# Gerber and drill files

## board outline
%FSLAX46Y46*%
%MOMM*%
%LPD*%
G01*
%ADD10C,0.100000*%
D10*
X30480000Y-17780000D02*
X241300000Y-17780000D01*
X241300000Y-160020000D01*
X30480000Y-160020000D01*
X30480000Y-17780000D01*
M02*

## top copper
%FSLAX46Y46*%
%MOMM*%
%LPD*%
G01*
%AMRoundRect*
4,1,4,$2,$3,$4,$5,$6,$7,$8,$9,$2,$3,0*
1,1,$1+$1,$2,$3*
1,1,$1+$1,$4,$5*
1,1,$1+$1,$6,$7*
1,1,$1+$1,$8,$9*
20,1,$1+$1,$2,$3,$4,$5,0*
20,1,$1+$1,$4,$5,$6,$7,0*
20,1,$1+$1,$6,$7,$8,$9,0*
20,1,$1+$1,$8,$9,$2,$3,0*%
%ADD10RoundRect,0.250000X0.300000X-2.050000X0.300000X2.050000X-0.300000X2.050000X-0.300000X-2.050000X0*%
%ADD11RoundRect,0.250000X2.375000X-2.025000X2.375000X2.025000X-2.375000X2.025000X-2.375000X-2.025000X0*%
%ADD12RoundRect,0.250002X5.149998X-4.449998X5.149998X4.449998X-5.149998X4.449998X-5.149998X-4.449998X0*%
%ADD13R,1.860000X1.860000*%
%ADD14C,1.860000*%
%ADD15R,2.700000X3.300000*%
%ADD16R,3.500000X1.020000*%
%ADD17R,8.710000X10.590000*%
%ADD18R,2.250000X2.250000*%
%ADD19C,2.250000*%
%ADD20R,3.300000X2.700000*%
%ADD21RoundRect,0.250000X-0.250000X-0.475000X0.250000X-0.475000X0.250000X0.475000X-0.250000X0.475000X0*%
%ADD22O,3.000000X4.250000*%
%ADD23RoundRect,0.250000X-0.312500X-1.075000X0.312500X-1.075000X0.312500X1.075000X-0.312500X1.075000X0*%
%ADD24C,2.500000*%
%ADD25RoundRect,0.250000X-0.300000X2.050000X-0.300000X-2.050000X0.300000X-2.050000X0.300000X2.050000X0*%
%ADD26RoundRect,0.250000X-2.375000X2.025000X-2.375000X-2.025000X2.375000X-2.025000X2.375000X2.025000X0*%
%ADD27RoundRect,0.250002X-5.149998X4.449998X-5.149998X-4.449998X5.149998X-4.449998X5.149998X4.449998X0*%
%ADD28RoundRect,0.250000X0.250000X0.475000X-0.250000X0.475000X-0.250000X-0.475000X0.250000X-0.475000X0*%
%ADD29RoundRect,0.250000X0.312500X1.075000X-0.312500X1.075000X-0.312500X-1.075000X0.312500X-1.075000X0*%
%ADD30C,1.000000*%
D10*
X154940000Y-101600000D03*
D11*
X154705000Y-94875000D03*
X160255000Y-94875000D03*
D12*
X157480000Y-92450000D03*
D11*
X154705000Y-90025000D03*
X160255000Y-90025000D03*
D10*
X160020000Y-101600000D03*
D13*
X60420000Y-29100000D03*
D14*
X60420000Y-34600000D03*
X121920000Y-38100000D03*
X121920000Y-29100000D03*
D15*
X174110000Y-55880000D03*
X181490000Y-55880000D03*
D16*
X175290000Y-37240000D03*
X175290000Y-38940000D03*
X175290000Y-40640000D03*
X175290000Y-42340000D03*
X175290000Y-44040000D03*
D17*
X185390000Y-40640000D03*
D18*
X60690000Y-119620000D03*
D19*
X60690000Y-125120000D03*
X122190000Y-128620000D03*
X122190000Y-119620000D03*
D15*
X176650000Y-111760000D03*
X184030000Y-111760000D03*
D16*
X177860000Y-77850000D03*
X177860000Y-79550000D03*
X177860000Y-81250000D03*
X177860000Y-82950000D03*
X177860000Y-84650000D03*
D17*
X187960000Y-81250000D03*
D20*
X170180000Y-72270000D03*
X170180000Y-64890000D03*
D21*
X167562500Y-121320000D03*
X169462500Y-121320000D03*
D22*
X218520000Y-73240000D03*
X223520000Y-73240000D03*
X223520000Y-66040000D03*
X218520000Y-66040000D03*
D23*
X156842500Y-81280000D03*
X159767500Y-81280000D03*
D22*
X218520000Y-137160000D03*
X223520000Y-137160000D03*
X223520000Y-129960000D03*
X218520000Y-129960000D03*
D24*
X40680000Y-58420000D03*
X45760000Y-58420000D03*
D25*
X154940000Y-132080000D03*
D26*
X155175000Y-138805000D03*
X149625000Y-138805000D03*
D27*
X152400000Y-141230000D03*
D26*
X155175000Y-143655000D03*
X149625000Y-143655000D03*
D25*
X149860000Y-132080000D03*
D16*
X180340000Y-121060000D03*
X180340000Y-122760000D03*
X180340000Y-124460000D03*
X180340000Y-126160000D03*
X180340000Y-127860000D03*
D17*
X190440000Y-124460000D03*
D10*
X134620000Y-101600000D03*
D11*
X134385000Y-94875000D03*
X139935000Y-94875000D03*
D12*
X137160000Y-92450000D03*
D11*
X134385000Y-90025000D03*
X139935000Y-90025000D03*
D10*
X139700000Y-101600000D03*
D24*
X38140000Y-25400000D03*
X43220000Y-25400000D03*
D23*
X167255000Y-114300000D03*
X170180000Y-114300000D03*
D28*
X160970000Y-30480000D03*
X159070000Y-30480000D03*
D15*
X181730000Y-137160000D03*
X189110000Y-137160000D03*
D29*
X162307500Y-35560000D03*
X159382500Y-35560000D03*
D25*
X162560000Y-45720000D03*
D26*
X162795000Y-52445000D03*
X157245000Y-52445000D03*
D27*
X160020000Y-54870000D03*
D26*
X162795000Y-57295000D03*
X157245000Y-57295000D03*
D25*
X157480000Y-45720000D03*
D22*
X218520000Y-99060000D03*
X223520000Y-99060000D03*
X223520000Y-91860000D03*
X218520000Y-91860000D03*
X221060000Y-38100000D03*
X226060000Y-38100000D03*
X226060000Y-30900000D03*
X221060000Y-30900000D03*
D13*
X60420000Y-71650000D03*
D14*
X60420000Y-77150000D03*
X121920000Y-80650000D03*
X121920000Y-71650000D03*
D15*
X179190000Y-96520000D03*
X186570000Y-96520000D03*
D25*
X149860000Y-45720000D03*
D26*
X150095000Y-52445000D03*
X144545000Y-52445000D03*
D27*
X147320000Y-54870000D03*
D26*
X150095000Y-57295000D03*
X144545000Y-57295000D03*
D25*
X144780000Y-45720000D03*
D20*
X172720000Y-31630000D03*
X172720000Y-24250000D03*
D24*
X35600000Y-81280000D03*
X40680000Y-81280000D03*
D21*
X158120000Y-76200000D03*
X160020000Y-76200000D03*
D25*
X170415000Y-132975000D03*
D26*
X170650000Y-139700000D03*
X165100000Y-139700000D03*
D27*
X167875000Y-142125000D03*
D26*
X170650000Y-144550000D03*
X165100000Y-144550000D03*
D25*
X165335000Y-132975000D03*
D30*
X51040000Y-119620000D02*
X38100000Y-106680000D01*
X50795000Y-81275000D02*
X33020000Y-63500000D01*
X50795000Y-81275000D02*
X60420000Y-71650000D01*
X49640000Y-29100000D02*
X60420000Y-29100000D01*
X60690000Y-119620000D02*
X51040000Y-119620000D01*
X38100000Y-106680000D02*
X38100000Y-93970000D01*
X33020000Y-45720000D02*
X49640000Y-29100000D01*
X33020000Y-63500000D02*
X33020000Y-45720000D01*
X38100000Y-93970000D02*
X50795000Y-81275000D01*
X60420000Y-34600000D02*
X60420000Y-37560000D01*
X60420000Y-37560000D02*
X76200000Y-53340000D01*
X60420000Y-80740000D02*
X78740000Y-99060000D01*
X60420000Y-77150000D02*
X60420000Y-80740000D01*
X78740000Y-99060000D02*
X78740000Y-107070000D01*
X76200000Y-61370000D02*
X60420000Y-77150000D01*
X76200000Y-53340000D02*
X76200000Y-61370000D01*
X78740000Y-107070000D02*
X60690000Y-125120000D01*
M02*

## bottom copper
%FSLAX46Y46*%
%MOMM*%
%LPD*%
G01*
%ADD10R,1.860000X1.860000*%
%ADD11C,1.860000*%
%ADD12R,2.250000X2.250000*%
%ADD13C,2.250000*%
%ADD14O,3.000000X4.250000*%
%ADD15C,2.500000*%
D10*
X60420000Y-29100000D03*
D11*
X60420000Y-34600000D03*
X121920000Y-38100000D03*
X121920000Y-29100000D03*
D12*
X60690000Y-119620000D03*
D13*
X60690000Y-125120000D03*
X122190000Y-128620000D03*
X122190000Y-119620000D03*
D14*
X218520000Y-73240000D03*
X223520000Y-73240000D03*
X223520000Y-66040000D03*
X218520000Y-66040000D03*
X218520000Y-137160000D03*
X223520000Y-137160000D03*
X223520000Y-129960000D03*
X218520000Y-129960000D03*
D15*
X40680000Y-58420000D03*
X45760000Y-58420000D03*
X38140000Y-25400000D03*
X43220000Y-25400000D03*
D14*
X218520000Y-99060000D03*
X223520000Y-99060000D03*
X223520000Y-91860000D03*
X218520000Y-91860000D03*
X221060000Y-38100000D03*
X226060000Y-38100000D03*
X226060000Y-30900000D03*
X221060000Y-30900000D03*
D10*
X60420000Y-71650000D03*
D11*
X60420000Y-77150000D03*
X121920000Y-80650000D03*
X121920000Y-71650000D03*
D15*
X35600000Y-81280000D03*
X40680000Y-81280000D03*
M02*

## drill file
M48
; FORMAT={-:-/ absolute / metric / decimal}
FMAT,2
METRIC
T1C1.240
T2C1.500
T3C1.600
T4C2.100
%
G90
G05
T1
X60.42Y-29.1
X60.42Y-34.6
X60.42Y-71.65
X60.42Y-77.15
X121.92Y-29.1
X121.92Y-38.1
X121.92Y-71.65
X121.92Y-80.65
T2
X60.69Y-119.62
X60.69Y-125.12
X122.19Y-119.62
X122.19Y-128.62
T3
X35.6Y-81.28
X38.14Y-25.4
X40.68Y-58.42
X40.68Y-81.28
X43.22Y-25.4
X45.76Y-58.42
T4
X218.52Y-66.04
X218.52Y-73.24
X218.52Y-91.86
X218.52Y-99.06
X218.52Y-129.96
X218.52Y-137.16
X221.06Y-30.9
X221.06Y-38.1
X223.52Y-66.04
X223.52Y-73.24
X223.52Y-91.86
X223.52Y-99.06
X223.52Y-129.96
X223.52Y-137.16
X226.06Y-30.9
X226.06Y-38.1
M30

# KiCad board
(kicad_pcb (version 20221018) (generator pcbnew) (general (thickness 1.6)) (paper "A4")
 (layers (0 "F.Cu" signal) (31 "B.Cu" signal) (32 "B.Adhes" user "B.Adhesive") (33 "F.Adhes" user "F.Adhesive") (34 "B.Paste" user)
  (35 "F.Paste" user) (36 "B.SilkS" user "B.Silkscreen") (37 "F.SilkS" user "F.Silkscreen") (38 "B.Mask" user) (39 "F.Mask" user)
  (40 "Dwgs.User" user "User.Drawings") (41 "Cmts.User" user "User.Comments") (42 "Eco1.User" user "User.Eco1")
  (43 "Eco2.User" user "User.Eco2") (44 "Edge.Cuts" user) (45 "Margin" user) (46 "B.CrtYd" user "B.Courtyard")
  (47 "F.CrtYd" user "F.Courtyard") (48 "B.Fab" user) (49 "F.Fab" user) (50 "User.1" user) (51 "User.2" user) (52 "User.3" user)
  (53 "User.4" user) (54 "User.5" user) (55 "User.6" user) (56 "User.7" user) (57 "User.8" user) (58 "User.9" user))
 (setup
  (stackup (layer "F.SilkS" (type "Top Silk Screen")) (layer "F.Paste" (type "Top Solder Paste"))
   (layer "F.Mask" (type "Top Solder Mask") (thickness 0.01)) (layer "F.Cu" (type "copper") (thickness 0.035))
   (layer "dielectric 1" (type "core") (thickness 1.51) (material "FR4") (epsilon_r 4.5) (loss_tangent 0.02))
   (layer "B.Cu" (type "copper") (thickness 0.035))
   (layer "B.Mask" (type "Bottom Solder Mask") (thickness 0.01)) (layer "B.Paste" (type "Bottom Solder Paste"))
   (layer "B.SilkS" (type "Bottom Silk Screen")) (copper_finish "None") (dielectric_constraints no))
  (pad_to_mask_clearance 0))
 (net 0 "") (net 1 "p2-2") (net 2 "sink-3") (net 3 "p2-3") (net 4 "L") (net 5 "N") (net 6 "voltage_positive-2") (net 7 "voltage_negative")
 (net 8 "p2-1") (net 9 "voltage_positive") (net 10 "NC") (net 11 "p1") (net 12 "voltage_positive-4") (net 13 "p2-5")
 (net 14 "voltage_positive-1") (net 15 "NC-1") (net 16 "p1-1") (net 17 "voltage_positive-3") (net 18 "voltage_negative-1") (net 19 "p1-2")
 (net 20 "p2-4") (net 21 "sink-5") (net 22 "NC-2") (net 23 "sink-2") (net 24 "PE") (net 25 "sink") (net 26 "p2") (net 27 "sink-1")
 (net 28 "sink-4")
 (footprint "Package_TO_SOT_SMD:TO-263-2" (layer "F.Cu") (at 157.48 93.95 90)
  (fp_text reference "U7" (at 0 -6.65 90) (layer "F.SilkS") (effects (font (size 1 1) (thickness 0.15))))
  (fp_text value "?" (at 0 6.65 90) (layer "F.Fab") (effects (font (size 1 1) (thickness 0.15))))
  (pad "1" smd roundrect (at -7.65 -2.54 90) (size 4.6 1.1) (layers "F.Cu" "F.Paste" "F.Mask") (roundrect_rratio 0.227273) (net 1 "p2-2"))
  (pad "2" smd roundrect (at -0.925 -2.775 90) (size 4.55 5.25) (layers "F.Cu" "F.Paste") (roundrect_rratio 0.054945) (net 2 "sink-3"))
  (pad "2" smd roundrect (at -0.925 2.775 90) (size 4.55 5.25) (layers "F.Cu" "F.Paste") (roundrect_rratio 0.054945) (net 2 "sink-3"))
  (pad "2" smd roundrect (at 1.5 0 90) (size 9.4 10.8) (layers "F.Cu" "F.Mask") (roundrect_rratio 0.026596) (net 2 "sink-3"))
  (pad "2" smd roundrect (at 3.925 -2.775 90) (size 4.55 5.25) (layers "F.Cu" "F.Paste") (roundrect_rratio 0.054945) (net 2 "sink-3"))
  (pad "2" smd roundrect (at 3.925 2.775 90) (size 4.55 5.25) (layers "F.Cu" "F.Paste") (roundrect_rratio 0.054945) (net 2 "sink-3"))
  (pad "3" smd roundrect (at -7.65 2.54 90) (size 4.6 1.1) (layers "F.Cu" "F.Paste" "F.Mask") (roundrect_rratio 0.227273) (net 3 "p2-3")))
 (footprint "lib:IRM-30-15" (layer "F.Cu") (at 91.17 44.1)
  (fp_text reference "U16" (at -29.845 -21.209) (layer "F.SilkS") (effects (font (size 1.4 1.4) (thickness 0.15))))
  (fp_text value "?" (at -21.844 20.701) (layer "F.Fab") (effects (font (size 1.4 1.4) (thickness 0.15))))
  (pad "1" thru_hole rect (at -30.75 -15) (size 1.86 1.86) (drill 1.24) (layers "*.Cu" "*.Mask") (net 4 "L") (solder_mask_margin 0.102))
  (pad "2" thru_hole circle (at -30.75 -9.5) (size 1.86 1.86) (drill 1.24) (layers "*.Cu" "*.Mask") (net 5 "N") (solder_mask_margin 0.102))
  (pad "3" thru_hole circle (at 30.75 -6) (size 1.86 1.86) (drill 1.24) (layers "*.Cu" "*.Mask") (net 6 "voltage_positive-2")
   (solder_mask_margin 0.102))
  (pad "4" thru_hole circle (at 30.75 -15) (size 1.86 1.86) (drill 1.24) (layers "*.Cu" "*.Mask") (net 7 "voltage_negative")
   (solder_mask_margin 0.102)))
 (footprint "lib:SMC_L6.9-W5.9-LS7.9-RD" (layer "F.Cu") (at 177.8 55.88)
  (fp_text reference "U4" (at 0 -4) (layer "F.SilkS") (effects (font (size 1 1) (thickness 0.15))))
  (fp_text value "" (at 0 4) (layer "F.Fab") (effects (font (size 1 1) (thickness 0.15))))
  (pad "1" smd rect (at -3.69 0) (size 2.7 3.3) (layers "F.Cu" "F.Paste" "F.Mask") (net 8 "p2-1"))
  (pad "2" smd rect (at 3.69 0) (size 2.7 3.3) (layers "F.Cu" "F.Paste" "F.Mask") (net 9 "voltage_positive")))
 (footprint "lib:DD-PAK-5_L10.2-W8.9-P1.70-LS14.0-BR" (layer "F.Cu") (at 180.34 40.64 180)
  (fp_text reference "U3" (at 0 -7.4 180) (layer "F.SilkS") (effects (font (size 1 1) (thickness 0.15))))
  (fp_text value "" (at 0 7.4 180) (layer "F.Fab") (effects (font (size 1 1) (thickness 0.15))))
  (pad "1" smd rect (at 5.05 3.4 180) (size 3.5 1.02) (layers "F.Cu" "F.Paste" "F.Mask") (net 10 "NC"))
  (pad "2" smd rect (at 5.05 1.7 180) (size 3.5 1.02) (layers "F.Cu" "F.Paste" "F.Mask") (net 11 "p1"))
  (pad "3" smd rect (at 5.05 0 180) (size 3.5 1.02) (layers "F.Cu" "F.Paste" "F.Mask") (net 9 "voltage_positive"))
  (pad "4" smd rect (at 5.05 -1.7 180) (size 3.5 1.02) (layers "F.Cu" "F.Paste" "F.Mask") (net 6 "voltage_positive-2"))
  (pad "5" smd rect (at 5.05 -3.4 180) (size 3.5 1.02) (layers "F.Cu" "F.Paste" "F.Mask") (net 8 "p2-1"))
  (pad "6" smd rect (at -5.05 0) (size 8.71 10.59) (layers "F.Cu" "F.Paste" "F.Mask") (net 9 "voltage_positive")))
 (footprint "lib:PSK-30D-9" (layer "F.Cu") (at 91.44 134.62)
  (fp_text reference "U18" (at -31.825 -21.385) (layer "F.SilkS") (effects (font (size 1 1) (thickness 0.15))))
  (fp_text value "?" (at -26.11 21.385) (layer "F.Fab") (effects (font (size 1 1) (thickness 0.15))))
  (pad "1" thru_hole rect (at -30.75 -15) (size 2.25 2.25) (drill 1.5) (layers "*.Cu" "*.Mask") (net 4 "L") (solder_mask_margin 0.102))
  (pad "2" thru_hole circle (at -30.75 -9.5) (size 2.25 2.25) (drill 1.5) (layers "*.Cu" "*.Mask") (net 5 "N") (solder_mask_margin 0.102))
  (pad "3" thru_hole circle (at 30.75 -6) (size 2.25 2.25) (drill 1.5) (layers "*.Cu" "*.Mask") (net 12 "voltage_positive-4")
   (solder_mask_margin 0.102))
  (pad "4" thru_hole circle (at 30.75 -15) (size 2.25 2.25) (drill 1.5) (layers "*.Cu" "*.Mask") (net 7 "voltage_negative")
   (solder_mask_margin 0.102)))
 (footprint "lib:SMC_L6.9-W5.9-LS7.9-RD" (layer "F.Cu") (at 180.34 111.76)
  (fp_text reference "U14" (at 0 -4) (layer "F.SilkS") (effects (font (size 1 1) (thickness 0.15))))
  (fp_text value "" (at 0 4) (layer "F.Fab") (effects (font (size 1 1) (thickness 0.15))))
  (pad "1" smd rect (at -3.69 0) (size 2.7 3.3) (layers "F.Cu" "F.Paste" "F.Mask") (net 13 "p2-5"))
  (pad "2" smd rect (at 3.69 0) (size 2.7 3.3) (layers "F.Cu" "F.Paste" "F.Mask") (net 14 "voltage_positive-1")))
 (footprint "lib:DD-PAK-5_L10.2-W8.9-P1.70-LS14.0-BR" (layer "F.Cu") (at 182.91 81.25 180)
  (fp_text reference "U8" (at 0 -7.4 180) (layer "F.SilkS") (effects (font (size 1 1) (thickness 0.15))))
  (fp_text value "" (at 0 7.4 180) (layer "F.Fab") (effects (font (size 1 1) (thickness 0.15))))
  (pad "1" smd rect (at 5.05 3.4 180) (size 3.5 1.02) (layers "F.Cu" "F.Paste" "F.Mask") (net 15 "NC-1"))
  (pad "2" smd rect (at 5.05 1.7 180) (size 3.5 1.02) (layers "F.Cu" "F.Paste" "F.Mask") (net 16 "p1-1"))
  (pad "3" smd rect (at 5.05 0 180) (size 3.5 1.02) (layers "F.Cu" "F.Paste" "F.Mask") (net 7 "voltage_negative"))
  (pad "4" smd rect (at 5.05 -1.7 180) (size 3.5 1.02) (layers "F.Cu" "F.Paste" "F.Mask") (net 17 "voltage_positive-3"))
  (pad "5" smd rect (at 5.05 -3.4 180) (size 3.5 1.02) (layers "F.Cu" "F.Paste" "F.Mask") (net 3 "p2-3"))
  (pad "6" smd rect (at -5.05 0) (size 8.71 10.59) (layers "F.Cu" "F.Paste" "F.Mask") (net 7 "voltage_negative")))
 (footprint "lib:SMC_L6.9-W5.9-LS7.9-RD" (layer "F.Cu") (at 170.18 68.58 90)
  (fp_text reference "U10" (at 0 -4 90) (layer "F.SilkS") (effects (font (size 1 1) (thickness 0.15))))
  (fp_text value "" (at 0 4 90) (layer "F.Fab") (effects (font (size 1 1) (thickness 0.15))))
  (pad "1" smd rect (at -3.69 0 90) (size 2.7 3.3) (layers "F.Cu" "F.Paste" "F.Mask") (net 7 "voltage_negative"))
  (pad "2" smd rect (at 3.69 0 90) (size 2.7 3.3) (layers "F.Cu" "F.Paste" "F.Mask") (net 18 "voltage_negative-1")))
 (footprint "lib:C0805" (layer "F.Cu") (at 168.5125 121.32)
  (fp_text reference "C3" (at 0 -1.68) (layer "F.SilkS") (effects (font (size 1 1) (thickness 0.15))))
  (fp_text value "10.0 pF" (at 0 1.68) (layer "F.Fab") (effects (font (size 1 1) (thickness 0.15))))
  (pad "1" smd roundrect (at -0.95 0) (size 1 1.45) (layers "F.Cu" "F.Paste" "F.Mask") (roundrect_rratio 0.25) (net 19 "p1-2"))
  (pad "2" smd roundrect (at 0.95 0) (size 1 1.45) (layers "F.Cu" "F.Paste" "F.Mask") (roundrect_rratio 0.25) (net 7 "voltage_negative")))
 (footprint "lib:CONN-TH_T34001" (layer "F.Cu") (at 221.02 69.64)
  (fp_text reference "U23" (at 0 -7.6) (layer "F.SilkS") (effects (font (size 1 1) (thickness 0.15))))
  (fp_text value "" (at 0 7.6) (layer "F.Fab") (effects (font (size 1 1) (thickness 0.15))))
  (pad "1" thru_hole oval (at -2.5 3.6) (size 3 4.25) (drill 2.100021) (layers "*.Cu" "*.Mask") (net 18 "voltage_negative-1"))
  (pad "2" thru_hole oval (at 2.5 3.6) (size 3 4.25) (drill 2.100021) (layers "*.Cu" "*.Mask") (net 18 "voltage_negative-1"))
  (pad "3" thru_hole oval (at 2.5 -3.6) (size 3 4.25) (drill 2.100021) (layers "*.Cu" "*.Mask") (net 18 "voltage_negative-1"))
  (pad "4" thru_hole oval (at -2.5 -3.6) (size 3 4.25) (drill 2.100021) (layers "*.Cu" "*.Mask") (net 18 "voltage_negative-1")))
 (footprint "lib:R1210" (layer "F.Cu") (at 158.305 81.28)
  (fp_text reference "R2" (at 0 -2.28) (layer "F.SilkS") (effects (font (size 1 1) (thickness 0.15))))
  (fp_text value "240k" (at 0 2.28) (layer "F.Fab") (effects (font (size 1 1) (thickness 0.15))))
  (pad "1" smd roundrect (at -1.4625 0) (size 1.125 2.65) (layers "F.Cu" "F.Paste" "F.Mask") (roundrect_rratio 0.222222) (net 16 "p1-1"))
  (pad "2" smd roundrect (at 1.4625 0) (size 1.125 2.65) (layers "F.Cu" "F.Paste" "F.Mask") (roundrect_rratio 0.222222)
   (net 18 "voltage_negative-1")))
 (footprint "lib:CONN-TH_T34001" (layer "F.Cu") (at 221.02 133.56)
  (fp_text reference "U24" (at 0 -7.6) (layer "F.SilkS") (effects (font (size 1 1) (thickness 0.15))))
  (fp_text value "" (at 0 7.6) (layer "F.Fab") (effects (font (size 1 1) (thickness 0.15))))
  (pad "1" thru_hole oval (at -2.5 3.6) (size 3 4.25) (drill 2.100021) (layers "*.Cu" "*.Mask") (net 14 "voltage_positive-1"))
  (pad "2" thru_hole oval (at 2.5 3.6) (size 3 4.25) (drill 2.100021) (layers "*.Cu" "*.Mask") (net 14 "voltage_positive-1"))
  (pad "3" thru_hole oval (at 2.5 -3.6) (size 3 4.25) (drill 2.100021) (layers "*.Cu" "*.Mask") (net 14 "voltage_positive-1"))
  (pad "4" thru_hole oval (at -2.5 -3.6) (size 3 4.25) (drill 2.100021) (layers "*.Cu" "*.Mask") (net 14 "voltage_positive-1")))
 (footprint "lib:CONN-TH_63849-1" (layer "F.Cu") (at 43.22 58.42)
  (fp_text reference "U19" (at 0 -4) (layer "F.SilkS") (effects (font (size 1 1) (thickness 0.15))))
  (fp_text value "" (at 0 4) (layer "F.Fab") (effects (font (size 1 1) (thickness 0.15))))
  (pad "1" thru_hole circle (at -2.54 0) (size 2.5 2.5) (drill 1.599997) (layers "*.Cu" "*.Mask") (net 4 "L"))
  (pad "1" thru_hole circle (at 2.54 0) (size 2.5 2.5) (drill 1.599997) (layers "*.Cu" "*.Mask") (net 4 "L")))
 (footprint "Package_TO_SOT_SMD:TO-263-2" (layer "F.Cu") (at 152.4 139.73 -90)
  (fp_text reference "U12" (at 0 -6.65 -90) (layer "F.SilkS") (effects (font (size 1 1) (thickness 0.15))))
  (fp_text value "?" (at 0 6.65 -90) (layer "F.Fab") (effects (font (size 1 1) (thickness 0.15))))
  (pad "1" smd roundrect (at -7.65 -2.54 270) (size 4.6 1.1) (layers "F.Cu" "F.Paste" "F.Mask") (roundrect_rratio 0.227273) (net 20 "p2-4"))
  (pad "2" smd roundrect (at -0.925 -2.775 270) (size 4.55 5.25) (layers "F.Cu" "F.Paste") (roundrect_rratio 0.054945) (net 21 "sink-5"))
  (pad "2" smd roundrect (at -0.925 2.775 270) (size 4.55 5.25) (layers "F.Cu" "F.Paste") (roundrect_rratio 0.054945) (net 21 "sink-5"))
  (pad "2" smd roundrect (at 1.5 0 270) (size 9.4 10.8) (layers "F.Cu" "F.Mask") (roundrect_rratio 0.026596) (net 21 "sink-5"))
  (pad "2" smd roundrect (at 3.925 -2.775 270) (size 4.55 5.25) (layers "F.Cu" "F.Paste") (roundrect_rratio 0.054945) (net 21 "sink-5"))
  (pad "2" smd roundrect (at 3.925 2.775 270) (size 4.55 5.25) (layers "F.Cu" "F.Paste") (roundrect_rratio 0.054945) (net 21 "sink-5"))
  (pad "3" smd roundrect (at -7.65 2.54 270) (size 4.6 1.1) (layers "F.Cu" "F.Paste" "F.Mask") (roundrect_rratio 0.227273) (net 13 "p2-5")))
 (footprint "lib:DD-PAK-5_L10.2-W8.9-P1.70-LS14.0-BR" (layer "F.Cu") (at 185.39 124.46 180)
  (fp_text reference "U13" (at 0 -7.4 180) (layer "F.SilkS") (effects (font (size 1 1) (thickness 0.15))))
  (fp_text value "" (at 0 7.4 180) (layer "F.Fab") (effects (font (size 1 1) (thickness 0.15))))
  (pad "1" smd rect (at 5.05 3.4 180) (size 3.5 1.02) (layers "F.Cu" "F.Paste" "F.Mask") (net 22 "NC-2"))
  (pad "2" smd rect (at 5.05 1.7 180) (size 3.5 1.02) (layers "F.Cu" "F.Paste" "F.Mask") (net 19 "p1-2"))
  (pad "3" smd rect (at 5.05 0 180) (size 3.5 1.02) (layers "F.Cu" "F.Paste" "F.Mask") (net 14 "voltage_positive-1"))
  (pad "4" smd rect (at 5.05 -1.7 180) (size 3.5 1.02) (layers "F.Cu" "F.Paste" "F.Mask") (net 12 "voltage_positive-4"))
  (pad "5" smd rect (at 5.05 -3.4 180) (size 3.5 1.02) (layers "F.Cu" "F.Paste" "F.Mask") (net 13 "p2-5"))
  (pad "6" smd rect (at -5.05 0) (size 8.71 10.59) (layers "F.Cu" "F.Paste" "F.Mask") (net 14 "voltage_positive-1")))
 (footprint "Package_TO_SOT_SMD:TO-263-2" (layer "F.Cu") (at 137.16 93.95 90)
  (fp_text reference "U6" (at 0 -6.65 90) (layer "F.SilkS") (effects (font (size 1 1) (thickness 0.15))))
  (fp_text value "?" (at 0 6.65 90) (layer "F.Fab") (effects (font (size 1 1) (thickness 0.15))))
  (pad "1" smd roundrect (at -7.65 -2.54 90) (size 4.6 1.1) (layers "F.Cu" "F.Paste" "F.Mask") (roundrect_rratio 0.227273)
   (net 17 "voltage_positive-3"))
  (pad "2" smd roundrect (at -0.925 -2.775 90) (size 4.55 5.25) (layers "F.Cu" "F.Paste") (roundrect_rratio 0.054945) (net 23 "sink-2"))
  (pad "2" smd roundrect (at -0.925 2.775 90) (size 4.55 5.25) (layers "F.Cu" "F.Paste") (roundrect_rratio 0.054945) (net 23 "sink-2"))
  (pad "2" smd roundrect (at 1.5 0 90) (size 9.4 10.8) (layers "F.Cu" "F.Mask") (roundrect_rratio 0.026596) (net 23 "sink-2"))
  (pad "2" smd roundrect (at 3.925 -2.775 90) (size 4.55 5.25) (layers "F.Cu" "F.Paste") (roundrect_rratio 0.054945) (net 23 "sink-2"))
  (pad "2" smd roundrect (at 3.925 2.775 90) (size 4.55 5.25) (layers "F.Cu" "F.Paste") (roundrect_rratio 0.054945) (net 23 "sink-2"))
  (pad "3" smd roundrect (at -7.65 2.54 90) (size 4.6 1.1) (layers "F.Cu" "F.Paste" "F.Mask") (roundrect_rratio 0.227273) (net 1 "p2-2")))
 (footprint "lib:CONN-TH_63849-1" (layer "F.Cu") (at 40.68 25.4)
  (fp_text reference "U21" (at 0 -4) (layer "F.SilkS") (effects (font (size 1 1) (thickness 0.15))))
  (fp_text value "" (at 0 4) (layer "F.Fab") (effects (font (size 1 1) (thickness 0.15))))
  (pad "1" thru_hole circle (at -2.54 0) (size 2.5 2.5) (drill 1.599997) (layers "*.Cu" "*.Mask") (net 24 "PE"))
  (pad "1" thru_hole circle (at 2.54 0) (size 2.5 2.5) (drill 1.599997) (layers "*.Cu" "*.Mask") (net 24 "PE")))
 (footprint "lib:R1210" (layer "F.Cu") (at 168.7175 114.3)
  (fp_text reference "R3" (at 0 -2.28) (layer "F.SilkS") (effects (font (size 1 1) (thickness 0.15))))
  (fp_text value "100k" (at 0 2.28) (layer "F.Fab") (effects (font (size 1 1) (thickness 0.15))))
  (pad "1" smd roundrect (at -1.4625 0) (size 1.125 2.65) (layers "F.Cu" "F.Paste" "F.Mask") (roundrect_rratio 0.222222) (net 19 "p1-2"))
  (pad "2" smd roundrect (at 1.4625 0) (size 1.125 2.65) (layers "F.Cu" "F.Paste" "F.Mask") (roundrect_rratio 0.222222)
   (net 7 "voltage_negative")))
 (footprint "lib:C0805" (layer "F.Cu") (at 160.02 30.48 180)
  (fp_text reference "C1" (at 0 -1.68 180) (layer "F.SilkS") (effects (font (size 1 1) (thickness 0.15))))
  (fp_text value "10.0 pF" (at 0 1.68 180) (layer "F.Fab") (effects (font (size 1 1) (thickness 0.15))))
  (pad "1" smd roundrect (at -0.95 0 180) (size 1 1.45) (layers "F.Cu" "F.Paste" "F.Mask") (roundrect_rratio 0.25) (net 11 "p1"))
  (pad "2" smd roundrect (at 0.95 0 180) (size 1 1.45) (layers "F.Cu" "F.Paste" "F.Mask") (roundrect_rratio 0.25) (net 7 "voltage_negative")))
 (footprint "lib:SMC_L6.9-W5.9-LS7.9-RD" (layer "F.Cu") (at 185.42 137.16)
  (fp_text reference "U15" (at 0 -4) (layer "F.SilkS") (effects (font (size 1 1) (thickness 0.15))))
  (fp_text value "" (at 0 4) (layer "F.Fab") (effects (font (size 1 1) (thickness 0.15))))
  (pad "1" smd rect (at -3.69 0) (size 2.7 3.3) (layers "F.Cu" "F.Paste" "F.Mask") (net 14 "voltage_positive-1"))
  (pad "2" smd rect (at 3.69 0) (size 2.7 3.3) (layers "F.Cu" "F.Paste" "F.Mask") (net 7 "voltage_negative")))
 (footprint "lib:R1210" (layer "F.Cu") (at 160.845 35.56 180)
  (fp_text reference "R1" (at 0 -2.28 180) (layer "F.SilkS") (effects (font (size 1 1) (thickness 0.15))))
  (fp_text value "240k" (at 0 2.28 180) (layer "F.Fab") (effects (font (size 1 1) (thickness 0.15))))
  (pad "1" smd roundrect (at -1.4625 0 180) (size 1.125 2.65) (layers "F.Cu" "F.Paste" "F.Mask") (roundrect_rratio 0.222222) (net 11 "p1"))
  (pad "2" smd roundrect (at 1.4625 0 180) (size 1.125 2.65) (layers "F.Cu" "F.Paste" "F.Mask") (roundrect_rratio 0.222222)
   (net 7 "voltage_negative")))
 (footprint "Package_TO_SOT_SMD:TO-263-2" (layer "F.Cu") (at 160.02 53.37 -90)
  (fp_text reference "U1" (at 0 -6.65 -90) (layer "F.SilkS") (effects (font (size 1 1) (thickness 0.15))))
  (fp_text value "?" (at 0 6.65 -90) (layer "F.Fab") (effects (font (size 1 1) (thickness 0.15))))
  (pad "1" smd roundrect (at -7.65 -2.54 270) (size 4.6 1.1) (layers "F.Cu" "F.Paste" "F.Mask") (roundrect_rratio 0.227273)
   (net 6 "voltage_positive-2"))
  (pad "2" smd roundrect (at -0.925 -2.775 270) (size 4.55 5.25) (layers "F.Cu" "F.Paste") (roundrect_rratio 0.054945) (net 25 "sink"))
  (pad "2" smd roundrect (at -0.925 2.775 270) (size 4.55 5.25) (layers "F.Cu" "F.Paste") (roundrect_rratio 0.054945) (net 25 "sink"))
  (pad "2" smd roundrect (at 1.5 0 270) (size 9.4 10.8) (layers "F.Cu" "F.Mask") (roundrect_rratio 0.026596) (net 25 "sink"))
  (pad "2" smd roundrect (at 3.925 -2.775 270) (size 4.55 5.25) (layers "F.Cu" "F.Paste") (roundrect_rratio 0.054945) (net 25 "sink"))
  (pad "2" smd roundrect (at 3.925 2.775 270) (size 4.55 5.25) (layers "F.Cu" "F.Paste") (roundrect_rratio 0.054945) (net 25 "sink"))
  (pad "3" smd roundrect (at -7.65 2.54 270) (size 4.6 1.1) (layers "F.Cu" "F.Paste" "F.Mask") (roundrect_rratio 0.227273) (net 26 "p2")))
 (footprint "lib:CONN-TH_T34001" (layer "F.Cu") (at 221.02 95.46)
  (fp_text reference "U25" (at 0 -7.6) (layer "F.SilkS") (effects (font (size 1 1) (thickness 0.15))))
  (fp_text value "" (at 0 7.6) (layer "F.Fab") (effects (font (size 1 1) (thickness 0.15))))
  (pad "1" thru_hole oval (at -2.5 3.6) (size 3 4.25) (drill 2.100021) (layers "*.Cu" "*.Mask") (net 7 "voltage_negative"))
  (pad "2" thru_hole oval (at 2.5 3.6) (size 3 4.25) (drill 2.100021) (layers "*.Cu" "*.Mask") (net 7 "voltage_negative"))
  (pad "3" thru_hole oval (at 2.5 -3.6) (size 3 4.25) (drill 2.100021) (layers "*.Cu" "*.Mask") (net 7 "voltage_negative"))
  (pad "4" thru_hole oval (at -2.5 -3.6) (size 3 4.25) (drill 2.100021) (layers "*.Cu" "*.Mask") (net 7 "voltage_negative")))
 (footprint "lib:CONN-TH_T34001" (layer "F.Cu") (at 223.56 34.5)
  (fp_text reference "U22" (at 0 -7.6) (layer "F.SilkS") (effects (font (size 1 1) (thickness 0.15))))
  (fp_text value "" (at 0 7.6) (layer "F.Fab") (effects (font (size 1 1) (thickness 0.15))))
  (pad "1" thru_hole oval (at -2.5 3.6) (size 3 4.25) (drill 2.100021) (layers "*.Cu" "*.Mask") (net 9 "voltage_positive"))
  (pad "2" thru_hole oval (at 2.5 3.6) (size 3 4.25) (drill 2.100021) (layers "*.Cu" "*.Mask") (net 9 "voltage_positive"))
  (pad "3" thru_hole oval (at 2.5 -3.6) (size 3 4.25) (drill 2.100021) (layers "*.Cu" "*.Mask") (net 9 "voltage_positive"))
  (pad "4" thru_hole oval (at -2.5 -3.6) (size 3 4.25) (drill 2.100021) (layers "*.Cu" "*.Mask") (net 9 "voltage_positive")))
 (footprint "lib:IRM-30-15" (layer "F.Cu") (at 91.17 86.65)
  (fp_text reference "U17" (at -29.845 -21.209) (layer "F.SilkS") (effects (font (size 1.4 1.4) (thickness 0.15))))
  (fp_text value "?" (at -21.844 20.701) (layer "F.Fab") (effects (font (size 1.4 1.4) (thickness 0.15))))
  (pad "1" thru_hole rect (at -30.75 -15) (size 1.86 1.86) (drill 1.24) (layers "*.Cu" "*.Mask") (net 4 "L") (solder_mask_margin 0.102))
  (pad "2" thru_hole circle (at -30.75 -9.5) (size 1.86 1.86) (drill 1.24) (layers "*.Cu" "*.Mask") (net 5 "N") (solder_mask_margin 0.102))
  (pad "3" thru_hole circle (at 30.75 -6) (size 1.86 1.86) (drill 1.24) (layers "*.Cu" "*.Mask") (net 17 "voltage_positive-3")
   (solder_mask_margin 0.102))
  (pad "4" thru_hole circle (at 30.75 -15) (size 1.86 1.86) (drill 1.24) (layers "*.Cu" "*.Mask") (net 18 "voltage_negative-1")
   (solder_mask_margin 0.102)))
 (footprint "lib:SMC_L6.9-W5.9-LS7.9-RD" (layer "F.Cu") (at 182.88 96.52)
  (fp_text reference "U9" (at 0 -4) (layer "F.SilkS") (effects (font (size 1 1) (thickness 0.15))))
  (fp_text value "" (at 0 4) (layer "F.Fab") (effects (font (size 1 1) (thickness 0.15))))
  (pad "1" smd rect (at -3.69 0) (size 2.7 3.3) (layers "F.Cu" "F.Paste" "F.Mask") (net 3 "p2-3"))
  (pad "2" smd rect (at 3.69 0) (size 2.7 3.3) (layers "F.Cu" "F.Paste" "F.Mask") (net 7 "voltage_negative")))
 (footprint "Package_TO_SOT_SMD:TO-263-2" (layer "F.Cu") (at 147.32 53.37 -90)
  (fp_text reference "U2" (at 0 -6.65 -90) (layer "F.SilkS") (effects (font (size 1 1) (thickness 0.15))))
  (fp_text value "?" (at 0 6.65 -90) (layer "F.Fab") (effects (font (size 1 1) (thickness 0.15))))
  (pad "1" smd roundrect (at -7.65 -2.54 270) (size 4.6 1.1) (layers "F.Cu" "F.Paste" "F.Mask") (roundrect_rratio 0.227273) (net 26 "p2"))
  (pad "2" smd roundrect (at -0.925 -2.775 270) (size 4.55 5.25) (layers "F.Cu" "F.Paste") (roundrect_rratio 0.054945) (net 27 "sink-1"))
  (pad "2" smd roundrect (at -0.925 2.775 270) (size 4.55 5.25) (layers "F.Cu" "F.Paste") (roundrect_rratio 0.054945) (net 27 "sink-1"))
  (pad "2" smd roundrect (at 1.5 0 270) (size 9.4 10.8) (layers "F.Cu" "F.Mask") (roundrect_rratio 0.026596) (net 27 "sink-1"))
  (pad "2" smd roundrect (at 3.925 -2.775 270) (size 4.55 5.25) (layers "F.Cu" "F.Paste") (roundrect_rratio 0.054945) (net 27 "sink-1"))
  (pad "2" smd roundrect (at 3.925 2.775 270) (size 4.55 5.25) (layers "F.Cu" "F.Paste") (roundrect_rratio 0.054945) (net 27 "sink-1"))
  (pad "3" smd roundrect (at -7.65 2.54 270) (size 4.6 1.1) (layers "F.Cu" "F.Paste" "F.Mask") (roundrect_rratio 0.227273) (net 8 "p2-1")))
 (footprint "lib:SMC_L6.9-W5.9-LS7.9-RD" (layer "F.Cu") (at 172.72 27.94 90)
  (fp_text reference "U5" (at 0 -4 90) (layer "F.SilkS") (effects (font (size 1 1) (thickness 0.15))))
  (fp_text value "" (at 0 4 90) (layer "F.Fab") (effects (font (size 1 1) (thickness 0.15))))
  (pad "1" smd rect (at -3.69 0 90) (size 2.7 3.3) (layers "F.Cu" "F.Paste" "F.Mask") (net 9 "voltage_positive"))
  (pad "2" smd rect (at 3.69 0 90) (size 2.7 3.3) (layers "F.Cu" "F.Paste" "F.Mask") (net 7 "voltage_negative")))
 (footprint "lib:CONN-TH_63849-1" (layer "F.Cu") (at 38.14 81.28)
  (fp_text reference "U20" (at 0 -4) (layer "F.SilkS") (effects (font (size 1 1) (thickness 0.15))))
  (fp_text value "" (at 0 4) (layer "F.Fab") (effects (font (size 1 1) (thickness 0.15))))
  (pad "1" thru_hole circle (at -2.54 0) (size 2.5 2.5) (drill 1.599997) (layers "*.Cu" "*.Mask") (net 5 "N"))
  (pad "1" thru_hole circle (at 2.54 0) (size 2.5 2.5) (drill 1.599997) (layers "*.Cu" "*.Mask") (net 5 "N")))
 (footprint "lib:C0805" (layer "F.Cu") (at 159.07 76.2)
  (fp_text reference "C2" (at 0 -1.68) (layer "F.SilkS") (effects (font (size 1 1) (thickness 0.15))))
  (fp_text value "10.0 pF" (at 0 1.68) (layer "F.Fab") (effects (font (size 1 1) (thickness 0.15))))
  (pad "1" smd roundrect (at -0.95 0) (size 1 1.45) (layers "F.Cu" "F.Paste" "F.Mask") (roundrect_rratio 0.25) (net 16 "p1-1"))
  (pad "2" smd roundrect (at 0.95 0) (size 1 1.45) (layers "F.Cu" "F.Paste" "F.Mask") (roundrect_rratio 0.25) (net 18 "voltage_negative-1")))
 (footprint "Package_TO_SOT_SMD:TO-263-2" (layer "F.Cu") (at 167.875 140.625 -90)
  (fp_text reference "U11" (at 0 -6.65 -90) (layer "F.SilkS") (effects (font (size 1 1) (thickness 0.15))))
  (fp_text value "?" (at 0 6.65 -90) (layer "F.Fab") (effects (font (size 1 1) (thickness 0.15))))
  (pad "1" smd roundrect (at -7.65 -2.54 270) (size 4.6 1.1) (layers "F.Cu" "F.Paste" "F.Mask") (roundrect_rratio 0.227273)
   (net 12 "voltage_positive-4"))
  (pad "2" smd roundrect (at -0.925 -2.775 270) (size 4.55 5.25) (layers "F.Cu" "F.Paste") (roundrect_rratio 0.054945) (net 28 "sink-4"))
  (pad "2" smd roundrect (at -0.925 2.775 270) (size 4.55 5.25) (layers "F.Cu" "F.Paste") (roundrect_rratio 0.054945) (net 28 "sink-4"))
  (pad "2" smd roundrect (at 1.5 0 270) (size 9.4 10.8) (layers "F.Cu" "F.Mask") (roundrect_rratio 0.026596) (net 28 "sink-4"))
  (pad "2" smd roundrect (at 3.925 -2.775 270) (size 4.55 5.25) (layers "F.Cu" "F.Paste") (roundrect_rratio 0.054945) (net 28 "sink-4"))
  (pad "2" smd roundrect (at 3.925 2.775 270) (size 4.55 5.25) (layers "F.Cu" "F.Paste") (roundrect_rratio 0.054945) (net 28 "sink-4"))
  (pad "3" smd roundrect (at -7.65 2.54 270) (size 4.6 1.1) (layers "F.Cu" "F.Paste" "F.Mask") (roundrect_rratio 0.227273) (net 20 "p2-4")))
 (gr_rect (start 30.48 17.78) (end 241.3 160.02) (stroke (width 0.1) (type default)) (fill none) (layer "Edge.Cuts"))
 (segment (start 51.04 119.62) (end 38.1 106.68) (width 1) (layer "F.Cu") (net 4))
 (segment (start 50.795 81.275) (end 33.02 63.5) (width 1) (layer "F.Cu") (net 4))
 (segment (start 50.795 81.275) (end 60.42 71.65) (width 1) (layer "F.Cu") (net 4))
 (segment (start 49.64 29.1) (end 60.42 29.1) (width 1) (layer "F.Cu") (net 4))
 (segment (start 60.69 119.62) (end 51.04 119.62) (width 1) (layer "F.Cu") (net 4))
 (segment (start 38.1 106.68) (end 38.1 93.97) (width 1) (layer "F.Cu") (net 4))
 (segment (start 33.02 45.72) (end 49.64 29.1) (width 1) (layer "F.Cu") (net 4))
 (segment (start 33.02 63.5) (end 33.02 45.72) (width 1) (layer "F.Cu") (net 4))
 (segment (start 38.1 93.97) (end 50.795 81.275) (width 1) (layer "F.Cu") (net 4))
 (segment (start 60.42 34.6) (end 60.42 37.56) (width 1) (layer "F.Cu") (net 5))
 (segment (start 60.42 37.56) (end 76.2 53.34) (width 1) (layer "F.Cu") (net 5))
 (segment (start 60.42 80.74) (end 78.74 99.06) (width 1) (layer "F.Cu") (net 5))
 (segment (start 60.42 77.15) (end 60.42 80.74) (width 1) (layer "F.Cu") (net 5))
 (segment (start 78.74 99.06) (end 78.74 107.07) (width 1) (layer "F.Cu") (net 5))
 (segment (start 76.2 61.37) (end 60.42 77.15) (width 1) (layer "F.Cu") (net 5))
 (segment (start 76.2 53.34) (end 76.2 61.37) (width 1) (layer "F.Cu") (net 5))
 (segment (start 78.74 107.07) (end 60.69 125.12) (width 1) (layer "F.Cu") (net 5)))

